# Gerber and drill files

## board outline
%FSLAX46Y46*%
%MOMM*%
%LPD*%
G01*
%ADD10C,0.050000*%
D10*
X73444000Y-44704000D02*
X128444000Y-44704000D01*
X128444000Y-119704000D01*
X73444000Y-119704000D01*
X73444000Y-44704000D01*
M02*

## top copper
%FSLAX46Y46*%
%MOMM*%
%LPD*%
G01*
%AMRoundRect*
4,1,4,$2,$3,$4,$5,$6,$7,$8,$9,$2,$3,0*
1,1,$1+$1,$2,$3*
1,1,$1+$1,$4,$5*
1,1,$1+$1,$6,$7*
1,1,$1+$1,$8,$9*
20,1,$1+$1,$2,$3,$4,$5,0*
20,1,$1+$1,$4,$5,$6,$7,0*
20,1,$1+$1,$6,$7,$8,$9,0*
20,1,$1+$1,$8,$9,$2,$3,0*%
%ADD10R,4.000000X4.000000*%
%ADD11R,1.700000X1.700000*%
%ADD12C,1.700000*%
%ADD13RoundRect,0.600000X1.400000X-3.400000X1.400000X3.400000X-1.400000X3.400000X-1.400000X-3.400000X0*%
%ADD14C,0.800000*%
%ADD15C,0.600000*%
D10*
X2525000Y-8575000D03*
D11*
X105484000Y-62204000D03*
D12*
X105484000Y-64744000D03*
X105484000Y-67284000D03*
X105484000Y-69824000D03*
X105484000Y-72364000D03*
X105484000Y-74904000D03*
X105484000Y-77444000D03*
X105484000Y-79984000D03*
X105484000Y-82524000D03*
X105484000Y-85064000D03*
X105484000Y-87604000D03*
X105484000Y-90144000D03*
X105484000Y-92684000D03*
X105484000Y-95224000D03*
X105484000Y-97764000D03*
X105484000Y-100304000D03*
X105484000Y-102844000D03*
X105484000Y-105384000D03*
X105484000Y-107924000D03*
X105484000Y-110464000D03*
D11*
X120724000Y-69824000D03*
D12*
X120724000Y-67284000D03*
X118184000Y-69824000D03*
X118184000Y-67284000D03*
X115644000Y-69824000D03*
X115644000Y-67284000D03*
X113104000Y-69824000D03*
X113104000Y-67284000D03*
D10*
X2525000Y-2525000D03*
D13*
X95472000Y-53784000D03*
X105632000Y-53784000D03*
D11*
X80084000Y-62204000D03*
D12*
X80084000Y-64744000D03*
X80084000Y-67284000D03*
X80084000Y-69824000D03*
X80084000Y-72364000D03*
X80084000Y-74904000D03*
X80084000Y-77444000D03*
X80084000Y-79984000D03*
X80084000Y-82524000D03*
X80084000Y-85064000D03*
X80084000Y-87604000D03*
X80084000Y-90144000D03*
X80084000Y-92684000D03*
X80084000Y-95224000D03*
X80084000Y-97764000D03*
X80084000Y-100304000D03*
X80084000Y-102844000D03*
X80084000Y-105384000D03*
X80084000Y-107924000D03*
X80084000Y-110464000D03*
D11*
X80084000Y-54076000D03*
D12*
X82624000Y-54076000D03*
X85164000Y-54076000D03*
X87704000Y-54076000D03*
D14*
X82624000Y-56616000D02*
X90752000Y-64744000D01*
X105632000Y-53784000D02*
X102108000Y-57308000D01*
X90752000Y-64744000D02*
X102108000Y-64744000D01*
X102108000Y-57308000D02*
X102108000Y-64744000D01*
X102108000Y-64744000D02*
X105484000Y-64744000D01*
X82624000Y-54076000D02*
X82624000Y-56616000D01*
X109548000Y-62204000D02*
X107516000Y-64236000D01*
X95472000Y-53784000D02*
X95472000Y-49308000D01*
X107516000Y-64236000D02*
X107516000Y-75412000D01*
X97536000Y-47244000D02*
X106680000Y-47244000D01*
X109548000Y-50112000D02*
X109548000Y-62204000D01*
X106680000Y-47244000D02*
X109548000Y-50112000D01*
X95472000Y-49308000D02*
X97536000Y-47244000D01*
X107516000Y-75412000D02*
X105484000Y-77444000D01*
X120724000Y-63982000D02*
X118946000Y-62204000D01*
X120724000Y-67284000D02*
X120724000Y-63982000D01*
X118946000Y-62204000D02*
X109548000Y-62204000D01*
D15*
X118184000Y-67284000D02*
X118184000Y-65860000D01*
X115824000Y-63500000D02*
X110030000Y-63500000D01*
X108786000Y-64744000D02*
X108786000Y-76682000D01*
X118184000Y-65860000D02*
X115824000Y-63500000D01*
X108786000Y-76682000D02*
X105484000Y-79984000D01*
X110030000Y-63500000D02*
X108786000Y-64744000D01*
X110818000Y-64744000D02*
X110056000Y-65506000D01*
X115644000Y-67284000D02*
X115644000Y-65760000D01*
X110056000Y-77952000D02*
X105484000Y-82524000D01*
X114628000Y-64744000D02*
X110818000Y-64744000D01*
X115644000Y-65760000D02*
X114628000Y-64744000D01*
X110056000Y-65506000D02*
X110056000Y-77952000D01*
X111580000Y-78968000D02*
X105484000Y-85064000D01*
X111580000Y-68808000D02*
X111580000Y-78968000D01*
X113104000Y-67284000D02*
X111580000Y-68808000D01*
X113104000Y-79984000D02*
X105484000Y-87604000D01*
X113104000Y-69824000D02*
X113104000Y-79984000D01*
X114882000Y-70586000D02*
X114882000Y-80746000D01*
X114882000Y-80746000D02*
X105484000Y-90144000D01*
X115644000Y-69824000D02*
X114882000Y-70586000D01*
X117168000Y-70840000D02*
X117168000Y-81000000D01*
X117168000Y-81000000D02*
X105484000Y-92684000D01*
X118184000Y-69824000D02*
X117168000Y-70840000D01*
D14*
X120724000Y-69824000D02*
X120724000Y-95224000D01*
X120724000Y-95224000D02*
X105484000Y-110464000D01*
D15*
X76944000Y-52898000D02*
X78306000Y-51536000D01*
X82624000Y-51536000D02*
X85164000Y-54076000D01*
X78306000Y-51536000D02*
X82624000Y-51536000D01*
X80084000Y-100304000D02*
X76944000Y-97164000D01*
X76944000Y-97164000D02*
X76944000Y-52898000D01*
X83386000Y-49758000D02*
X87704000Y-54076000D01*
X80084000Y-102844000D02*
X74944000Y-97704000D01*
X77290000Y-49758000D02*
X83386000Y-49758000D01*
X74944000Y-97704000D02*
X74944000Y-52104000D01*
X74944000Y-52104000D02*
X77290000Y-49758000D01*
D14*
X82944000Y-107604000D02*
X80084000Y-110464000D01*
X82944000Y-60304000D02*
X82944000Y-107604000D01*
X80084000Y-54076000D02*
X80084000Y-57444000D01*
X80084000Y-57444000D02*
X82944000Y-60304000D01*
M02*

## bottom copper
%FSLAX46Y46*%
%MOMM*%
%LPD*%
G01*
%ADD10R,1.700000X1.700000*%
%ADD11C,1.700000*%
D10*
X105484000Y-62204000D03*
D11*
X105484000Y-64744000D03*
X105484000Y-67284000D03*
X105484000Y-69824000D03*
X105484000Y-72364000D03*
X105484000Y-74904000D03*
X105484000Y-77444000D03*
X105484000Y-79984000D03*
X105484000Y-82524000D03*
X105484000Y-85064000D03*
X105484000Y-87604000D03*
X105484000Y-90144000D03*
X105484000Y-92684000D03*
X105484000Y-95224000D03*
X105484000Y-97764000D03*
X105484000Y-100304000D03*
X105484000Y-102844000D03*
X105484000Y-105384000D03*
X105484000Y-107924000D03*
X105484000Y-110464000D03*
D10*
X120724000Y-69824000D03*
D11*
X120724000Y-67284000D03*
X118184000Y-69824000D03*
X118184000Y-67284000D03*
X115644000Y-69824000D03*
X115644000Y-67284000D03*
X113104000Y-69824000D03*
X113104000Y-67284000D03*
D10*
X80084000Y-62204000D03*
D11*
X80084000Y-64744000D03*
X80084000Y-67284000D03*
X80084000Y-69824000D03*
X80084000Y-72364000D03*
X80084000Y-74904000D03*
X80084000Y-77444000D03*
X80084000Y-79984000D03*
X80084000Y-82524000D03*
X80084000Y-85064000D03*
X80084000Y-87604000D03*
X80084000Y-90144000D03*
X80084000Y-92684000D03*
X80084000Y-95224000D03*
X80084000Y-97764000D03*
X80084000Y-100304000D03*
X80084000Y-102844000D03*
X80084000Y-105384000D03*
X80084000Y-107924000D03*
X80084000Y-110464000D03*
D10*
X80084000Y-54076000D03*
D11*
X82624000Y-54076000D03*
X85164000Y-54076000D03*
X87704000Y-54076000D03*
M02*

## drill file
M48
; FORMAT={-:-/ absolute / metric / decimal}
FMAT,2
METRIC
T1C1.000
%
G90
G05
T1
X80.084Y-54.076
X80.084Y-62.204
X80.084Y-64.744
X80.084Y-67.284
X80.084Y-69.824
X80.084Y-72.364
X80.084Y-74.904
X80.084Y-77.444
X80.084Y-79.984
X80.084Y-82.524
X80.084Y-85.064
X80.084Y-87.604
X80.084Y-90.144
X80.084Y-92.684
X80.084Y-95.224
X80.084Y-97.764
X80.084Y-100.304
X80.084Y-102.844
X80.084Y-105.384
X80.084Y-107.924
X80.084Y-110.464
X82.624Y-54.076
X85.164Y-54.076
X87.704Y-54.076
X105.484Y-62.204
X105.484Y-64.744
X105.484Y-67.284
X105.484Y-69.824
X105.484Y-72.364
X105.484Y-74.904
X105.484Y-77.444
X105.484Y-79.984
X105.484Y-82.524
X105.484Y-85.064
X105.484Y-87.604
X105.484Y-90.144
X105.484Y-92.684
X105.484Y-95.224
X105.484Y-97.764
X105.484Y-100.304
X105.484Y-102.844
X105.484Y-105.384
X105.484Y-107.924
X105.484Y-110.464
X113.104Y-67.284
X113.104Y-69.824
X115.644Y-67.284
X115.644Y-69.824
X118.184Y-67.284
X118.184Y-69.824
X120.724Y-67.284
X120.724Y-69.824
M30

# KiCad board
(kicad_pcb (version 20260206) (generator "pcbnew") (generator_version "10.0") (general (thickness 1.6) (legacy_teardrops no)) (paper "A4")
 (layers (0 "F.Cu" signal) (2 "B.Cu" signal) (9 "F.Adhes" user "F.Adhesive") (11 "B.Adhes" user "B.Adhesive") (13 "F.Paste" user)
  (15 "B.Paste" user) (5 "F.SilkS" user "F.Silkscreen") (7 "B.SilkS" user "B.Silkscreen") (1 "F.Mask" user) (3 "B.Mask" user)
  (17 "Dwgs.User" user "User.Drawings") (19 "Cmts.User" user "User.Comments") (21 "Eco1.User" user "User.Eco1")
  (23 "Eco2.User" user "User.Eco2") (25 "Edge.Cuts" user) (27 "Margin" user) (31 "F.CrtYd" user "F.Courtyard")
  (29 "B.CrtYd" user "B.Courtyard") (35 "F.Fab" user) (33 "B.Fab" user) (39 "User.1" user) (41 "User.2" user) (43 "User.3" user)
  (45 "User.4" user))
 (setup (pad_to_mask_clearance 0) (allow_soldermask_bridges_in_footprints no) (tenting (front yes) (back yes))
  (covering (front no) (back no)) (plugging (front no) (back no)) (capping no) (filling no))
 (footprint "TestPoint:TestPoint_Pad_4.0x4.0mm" (layer "F.Cu") (at 2.525 8.575)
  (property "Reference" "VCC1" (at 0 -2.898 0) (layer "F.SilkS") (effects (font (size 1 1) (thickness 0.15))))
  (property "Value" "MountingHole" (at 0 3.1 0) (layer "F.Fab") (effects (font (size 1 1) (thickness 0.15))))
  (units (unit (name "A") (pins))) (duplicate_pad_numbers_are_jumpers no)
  (pad "1" smd rect (at 0 0) (size 4 4) (layers "F.Cu" "F.Mask")))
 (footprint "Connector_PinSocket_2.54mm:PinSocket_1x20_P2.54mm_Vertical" (layer "F.Cu") (at 105.484 62.204)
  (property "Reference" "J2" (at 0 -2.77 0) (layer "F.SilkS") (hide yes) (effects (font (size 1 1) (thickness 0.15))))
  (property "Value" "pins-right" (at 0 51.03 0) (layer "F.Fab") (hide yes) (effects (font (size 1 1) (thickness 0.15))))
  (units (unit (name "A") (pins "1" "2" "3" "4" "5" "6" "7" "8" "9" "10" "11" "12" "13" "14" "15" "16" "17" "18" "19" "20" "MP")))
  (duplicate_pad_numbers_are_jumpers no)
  (pad "1" thru_hole rect (at 0 0) (size 1.7 1.7) (drill 1) (layers "*.Cu" "*.Mask") (remove_unused_layers no)
   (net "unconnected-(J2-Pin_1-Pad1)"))
  (pad "2" thru_hole circle (at 0 2.54) (size 1.7 1.7) (drill 1) (layers "*.Cu" "*.Mask") (remove_unused_layers no) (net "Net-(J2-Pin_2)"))
  (pad "3" thru_hole circle (at 0 5.08) (size 1.7 1.7) (drill 1) (layers "*.Cu" "*.Mask") (remove_unused_layers no)
   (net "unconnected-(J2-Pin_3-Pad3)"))
  (pad "4" thru_hole circle (at 0 7.62) (size 1.7 1.7) (drill 1) (layers "*.Cu" "*.Mask") (remove_unused_layers no)
   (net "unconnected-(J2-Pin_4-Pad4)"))
  (pad "5" thru_hole circle (at 0 10.16) (size 1.7 1.7) (drill 1) (layers "*.Cu" "*.Mask") (remove_unused_layers no)
   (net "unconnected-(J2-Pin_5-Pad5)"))
  (pad "6" thru_hole circle (at 0 12.7) (size 1.7 1.7) (drill 1) (layers "*.Cu" "*.Mask") (remove_unused_layers no)
   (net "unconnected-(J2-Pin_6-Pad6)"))
  (pad "7" thru_hole circle (at 0 15.24) (size 1.7 1.7) (drill 1) (layers "*.Cu" "*.Mask") (remove_unused_layers no) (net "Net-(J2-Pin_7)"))
  (pad "8" thru_hole circle (at 0 17.78) (size 1.7 1.7) (drill 1) (layers "*.Cu" "*.Mask") (remove_unused_layers no) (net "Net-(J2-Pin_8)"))
  (pad "9" thru_hole circle (at 0 20.32) (size 1.7 1.7) (drill 1) (layers "*.Cu" "*.Mask") (remove_unused_layers no) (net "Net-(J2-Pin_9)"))
  (pad "10" thru_hole circle (at 0 22.86) (size 1.7 1.7) (drill 1) (layers "*.Cu" "*.Mask") (remove_unused_layers no)
   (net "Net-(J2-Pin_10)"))
  (pad "11" thru_hole circle (at 0 25.4) (size 1.7 1.7) (drill 1) (layers "*.Cu" "*.Mask") (remove_unused_layers no) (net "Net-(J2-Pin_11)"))
  (pad "12" thru_hole circle (at 0 27.94) (size 1.7 1.7) (drill 1) (layers "*.Cu" "*.Mask") (remove_unused_layers no)
   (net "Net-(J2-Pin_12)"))
  (pad "13" thru_hole circle (at 0 30.48) (size 1.7 1.7) (drill 1) (layers "*.Cu" "*.Mask") (remove_unused_layers no)
   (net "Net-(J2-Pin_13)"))
  (pad "14" thru_hole circle (at 0 33.02) (size 1.7 1.7) (drill 1) (layers "*.Cu" "*.Mask") (remove_unused_layers no)
   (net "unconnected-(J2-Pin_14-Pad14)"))
  (pad "15" thru_hole circle (at 0 35.56) (size 1.7 1.7) (drill 1) (layers "*.Cu" "*.Mask") (remove_unused_layers no)
   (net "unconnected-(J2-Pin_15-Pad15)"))
  (pad "16" thru_hole circle (at 0 38.1) (size 1.7 1.7) (drill 1) (layers "*.Cu" "*.Mask") (remove_unused_layers no)
   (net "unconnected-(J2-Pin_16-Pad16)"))
  (pad "17" thru_hole circle (at 0 40.64) (size 1.7 1.7) (drill 1) (layers "*.Cu" "*.Mask") (remove_unused_layers no)
   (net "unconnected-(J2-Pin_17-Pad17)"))
  (pad "18" thru_hole circle (at 0 43.18) (size 1.7 1.7) (drill 1) (layers "*.Cu" "*.Mask") (remove_unused_layers no)
   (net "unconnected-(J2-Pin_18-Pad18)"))
  (pad "19" thru_hole circle (at 0 45.72) (size 1.7 1.7) (drill 1) (layers "*.Cu" "*.Mask") (remove_unused_layers no)
   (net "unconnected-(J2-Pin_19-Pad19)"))
  (pad "20" thru_hole circle (at 0 48.26) (size 1.7 1.7) (drill 1) (layers "*.Cu" "*.Mask") (remove_unused_layers no)
   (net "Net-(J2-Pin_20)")))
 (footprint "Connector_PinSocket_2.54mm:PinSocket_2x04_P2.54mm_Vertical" (layer "F.Cu") (at 120.724 69.824 -90)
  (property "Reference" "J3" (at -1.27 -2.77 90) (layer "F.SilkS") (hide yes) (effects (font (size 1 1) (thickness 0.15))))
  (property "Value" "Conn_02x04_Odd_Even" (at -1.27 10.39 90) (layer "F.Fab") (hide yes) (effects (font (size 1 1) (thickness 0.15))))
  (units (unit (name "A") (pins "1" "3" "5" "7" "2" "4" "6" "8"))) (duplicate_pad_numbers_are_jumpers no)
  (pad "1" thru_hole rect (at 0 0 270) (size 1.7 1.7) (drill 1) (layers "*.Cu" "*.Mask") (remove_unused_layers no) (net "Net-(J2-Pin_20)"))
  (pad "2" thru_hole circle (at -2.54 0 270) (size 1.7 1.7) (drill 1) (layers "*.Cu" "*.Mask") (remove_unused_layers no)
   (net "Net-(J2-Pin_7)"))
  (pad "3" thru_hole circle (at 0 2.54 270) (size 1.7 1.7) (drill 1) (layers "*.Cu" "*.Mask") (remove_unused_layers no)
   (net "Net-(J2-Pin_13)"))
  (pad "4" thru_hole circle (at -2.54 2.54 270) (size 1.7 1.7) (drill 1) (layers "*.Cu" "*.Mask") (remove_unused_layers no)
   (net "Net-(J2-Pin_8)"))
  (pad "5" thru_hole circle (at 0 5.08 270) (size 1.7 1.7) (drill 1) (layers "*.Cu" "*.Mask") (remove_unused_layers no)
   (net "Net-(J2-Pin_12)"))
  (pad "6" thru_hole circle (at -2.54 5.08 270) (size 1.7 1.7) (drill 1) (layers "*.Cu" "*.Mask") (remove_unused_layers no)
   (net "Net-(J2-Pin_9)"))
  (pad "7" thru_hole circle (at 0 7.62 270) (size 1.7 1.7) (drill 1) (layers "*.Cu" "*.Mask") (remove_unused_layers no)
   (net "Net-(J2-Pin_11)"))
  (pad "8" thru_hole circle (at -2.54 7.62 270) (size 1.7 1.7) (drill 1) (layers "*.Cu" "*.Mask") (remove_unused_layers no)
   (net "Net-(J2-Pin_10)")))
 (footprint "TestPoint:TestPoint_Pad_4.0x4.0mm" (layer "F.Cu") (at 2.525 2.525)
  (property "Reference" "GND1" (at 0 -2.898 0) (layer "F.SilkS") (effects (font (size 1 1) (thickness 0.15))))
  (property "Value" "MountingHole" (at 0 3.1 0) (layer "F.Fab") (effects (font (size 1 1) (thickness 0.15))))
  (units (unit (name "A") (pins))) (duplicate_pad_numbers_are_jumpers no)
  (pad "1" smd rect (at 0 0) (size 4 4) (layers "F.Cu" "F.Mask")))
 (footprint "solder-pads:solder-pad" (layer "F.Cu") (at 100.552 53.784)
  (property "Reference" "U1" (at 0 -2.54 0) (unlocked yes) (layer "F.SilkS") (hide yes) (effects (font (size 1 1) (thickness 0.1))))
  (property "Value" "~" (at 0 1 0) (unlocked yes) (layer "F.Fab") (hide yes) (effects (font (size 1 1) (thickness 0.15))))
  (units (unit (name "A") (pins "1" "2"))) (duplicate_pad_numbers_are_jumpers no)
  (pad "1" smd roundrect (at -5.08 0 90) (size 8 4) (layers "F.Cu" "F.Mask" "F.Paste") (roundrect_rratio 0.15) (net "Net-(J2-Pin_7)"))
  (pad "2" smd roundrect (at 5.08 0 90) (size 8 4) (layers "F.Cu" "F.Mask" "F.Paste") (roundrect_rratio 0.15) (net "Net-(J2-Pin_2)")))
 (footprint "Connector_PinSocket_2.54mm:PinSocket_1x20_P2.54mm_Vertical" (layer "F.Cu") (at 80.084 62.204)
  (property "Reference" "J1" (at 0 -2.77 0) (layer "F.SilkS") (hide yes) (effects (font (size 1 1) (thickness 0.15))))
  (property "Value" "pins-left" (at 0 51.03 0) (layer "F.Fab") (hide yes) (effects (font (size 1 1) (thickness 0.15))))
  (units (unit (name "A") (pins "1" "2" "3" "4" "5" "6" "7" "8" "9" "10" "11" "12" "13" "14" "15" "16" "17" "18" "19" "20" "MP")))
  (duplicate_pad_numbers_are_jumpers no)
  (pad "1" thru_hole rect (at 0 0) (size 1.7 1.7) (drill 1) (layers "*.Cu" "*.Mask") (remove_unused_layers no)
   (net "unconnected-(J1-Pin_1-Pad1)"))
  (pad "2" thru_hole circle (at 0 2.54) (size 1.7 1.7) (drill 1) (layers "*.Cu" "*.Mask") (remove_unused_layers no)
   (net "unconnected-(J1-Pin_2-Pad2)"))
  (pad "3" thru_hole circle (at 0 5.08) (size 1.7 1.7) (drill 1) (layers "*.Cu" "*.Mask") (remove_unused_layers no)
   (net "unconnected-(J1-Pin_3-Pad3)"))
  (pad "4" thru_hole circle (at 0 7.62) (size 1.7 1.7) (drill 1) (layers "*.Cu" "*.Mask") (remove_unused_layers no)
   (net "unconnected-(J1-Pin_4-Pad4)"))
  (pad "5" thru_hole circle (at 0 10.16) (size 1.7 1.7) (drill 1) (layers "*.Cu" "*.Mask") (remove_unused_layers no)
   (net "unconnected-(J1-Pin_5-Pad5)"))
  (pad "6" thru_hole circle (at 0 12.7) (size 1.7 1.7) (drill 1) (layers "*.Cu" "*.Mask") (remove_unused_layers no)
   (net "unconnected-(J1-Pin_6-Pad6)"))
  (pad "7" thru_hole circle (at 0 15.24) (size 1.7 1.7) (drill 1) (layers "*.Cu" "*.Mask") (remove_unused_layers no)
   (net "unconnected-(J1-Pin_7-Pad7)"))
  (pad "8" thru_hole circle (at 0 17.78) (size 1.7 1.7) (drill 1) (layers "*.Cu" "*.Mask") (remove_unused_layers no)
   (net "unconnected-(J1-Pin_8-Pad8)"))
  (pad "9" thru_hole circle (at 0 20.32) (size 1.7 1.7) (drill 1) (layers "*.Cu" "*.Mask") (remove_unused_layers no)
   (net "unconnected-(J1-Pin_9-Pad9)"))
  (pad "10" thru_hole circle (at 0 22.86) (size 1.7 1.7) (drill 1) (layers "*.Cu" "*.Mask") (remove_unused_layers no)
   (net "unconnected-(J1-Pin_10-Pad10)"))
  (pad "11" thru_hole circle (at 0 25.4) (size 1.7 1.7) (drill 1) (layers "*.Cu" "*.Mask") (remove_unused_layers no)
   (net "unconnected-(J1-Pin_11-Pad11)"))
  (pad "12" thru_hole circle (at 0 27.94) (size 1.7 1.7) (drill 1) (layers "*.Cu" "*.Mask") (remove_unused_layers no)
   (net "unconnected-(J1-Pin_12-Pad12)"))
  (pad "13" thru_hole circle (at 0 30.48) (size 1.7 1.7) (drill 1) (layers "*.Cu" "*.Mask") (remove_unused_layers no)
   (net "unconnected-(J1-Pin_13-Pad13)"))
  (pad "14" thru_hole circle (at 0 33.02) (size 1.7 1.7) (drill 1) (layers "*.Cu" "*.Mask") (remove_unused_layers no)
   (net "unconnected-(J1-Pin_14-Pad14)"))
  (pad "15" thru_hole circle (at 0 35.56) (size 1.7 1.7) (drill 1) (layers "*.Cu" "*.Mask") (remove_unused_layers no)
   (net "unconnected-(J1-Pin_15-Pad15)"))
  (pad "16" thru_hole circle (at 0 38.1) (size 1.7 1.7) (drill 1) (layers "*.Cu" "*.Mask") (remove_unused_layers no) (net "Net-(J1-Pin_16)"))
  (pad "17" thru_hole circle (at 0 40.64) (size 1.7 1.7) (drill 1) (layers "*.Cu" "*.Mask") (remove_unused_layers no)
   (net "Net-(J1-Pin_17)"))
  (pad "18" thru_hole circle (at 0 43.18) (size 1.7 1.7) (drill 1) (layers "*.Cu" "*.Mask") (remove_unused_layers no)
   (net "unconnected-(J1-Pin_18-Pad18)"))
  (pad "19" thru_hole circle (at 0 45.72) (size 1.7 1.7) (drill 1) (layers "*.Cu" "*.Mask") (remove_unused_layers no)
   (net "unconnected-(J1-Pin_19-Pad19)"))
  (pad "20" thru_hole circle (at 0 48.26) (size 1.7 1.7) (drill 1) (layers "*.Cu" "*.Mask") (remove_unused_layers no)
   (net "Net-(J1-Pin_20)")))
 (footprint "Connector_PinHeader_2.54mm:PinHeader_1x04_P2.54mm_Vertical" (layer "F.Cu") (at 80.084 54.076 90)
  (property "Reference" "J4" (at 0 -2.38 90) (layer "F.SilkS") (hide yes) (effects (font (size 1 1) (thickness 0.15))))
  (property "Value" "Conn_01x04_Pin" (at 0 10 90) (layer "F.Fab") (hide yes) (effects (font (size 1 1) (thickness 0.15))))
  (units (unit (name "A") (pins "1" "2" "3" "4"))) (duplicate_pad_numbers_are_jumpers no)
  (pad "1" thru_hole rect (at 0 0 90) (size 1.7 1.7) (drill 1) (layers "*.Cu" "*.Mask") (remove_unused_layers no) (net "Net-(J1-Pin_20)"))
  (pad "2" thru_hole circle (at 0 2.54 90) (size 1.7 1.7) (drill 1) (layers "*.Cu" "*.Mask") (remove_unused_layers no)
   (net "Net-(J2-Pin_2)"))
  (pad "3" thru_hole circle (at 0 5.08 90) (size 1.7 1.7) (drill 1) (layers "*.Cu" "*.Mask") (remove_unused_layers no)
   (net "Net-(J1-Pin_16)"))
  (pad "4" thru_hole circle (at 0 7.62 90) (size 1.7 1.7) (drill 1) (layers "*.Cu" "*.Mask") (remove_unused_layers no)
   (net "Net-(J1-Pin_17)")))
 (gr_rect (start 73.444 44.704) (end 128.444 119.704) (stroke (width 0.05) (type default)) (fill no) (layer "Edge.Cuts"))
 (segment (start 82.624 56.616) (end 90.752 64.744) (width 0.8) (layer "F.Cu") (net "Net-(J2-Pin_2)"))
 (segment (start 105.632 53.784) (end 102.108 57.308) (width 0.8) (layer "F.Cu") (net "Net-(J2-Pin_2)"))
 (segment (start 90.752 64.744) (end 102.108 64.744) (width 0.8) (layer "F.Cu") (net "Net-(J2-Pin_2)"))
 (segment (start 102.108 57.308) (end 102.108 64.744) (width 0.8) (layer "F.Cu") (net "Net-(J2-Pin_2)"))
 (segment (start 102.108 64.744) (end 105.484 64.744) (width 0.8) (layer "F.Cu") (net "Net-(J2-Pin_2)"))
 (segment (start 82.624 54.076) (end 82.624 56.616) (width 0.8) (layer "F.Cu") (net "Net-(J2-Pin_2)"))
 (segment (start 109.548 62.204) (end 107.516 64.236) (width 0.8) (layer "F.Cu") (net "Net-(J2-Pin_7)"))
 (segment (start 95.472 53.784) (end 95.472 49.308) (width 0.8) (layer "F.Cu") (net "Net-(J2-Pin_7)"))
 (segment (start 107.516 64.236) (end 107.516 75.412) (width 0.8) (layer "F.Cu") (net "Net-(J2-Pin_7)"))
 (segment (start 97.536 47.244) (end 106.68 47.244) (width 0.8) (layer "F.Cu") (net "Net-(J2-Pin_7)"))
 (segment (start 109.548 50.112) (end 109.548 62.204) (width 0.8) (layer "F.Cu") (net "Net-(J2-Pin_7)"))
 (segment (start 106.68 47.244) (end 109.548 50.112) (width 0.8) (layer "F.Cu") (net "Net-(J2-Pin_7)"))
 (segment (start 95.472 49.308) (end 97.536 47.244) (width 0.8) (layer "F.Cu") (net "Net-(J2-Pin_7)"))
 (segment (start 107.516 75.412) (end 105.484 77.444) (width 0.8) (layer "F.Cu") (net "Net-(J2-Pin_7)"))
 (segment (start 120.724 63.982) (end 118.946 62.204) (width 0.8) (layer "F.Cu") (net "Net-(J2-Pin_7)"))
 (segment (start 120.724 67.284) (end 120.724 63.982) (width 0.8) (layer "F.Cu") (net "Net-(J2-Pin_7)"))
 (segment (start 118.946 62.204) (end 109.548 62.204) (width 0.8) (layer "F.Cu") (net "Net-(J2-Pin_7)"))
 (segment (start 118.184 67.284) (end 118.184 65.86) (width 0.6) (layer "F.Cu") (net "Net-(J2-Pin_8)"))
 (segment (start 115.824 63.5) (end 110.03 63.5) (width 0.6) (layer "F.Cu") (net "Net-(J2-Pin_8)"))
 (segment (start 108.786 64.744) (end 108.786 76.682) (width 0.6) (layer "F.Cu") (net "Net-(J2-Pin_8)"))
 (segment (start 118.184 65.86) (end 115.824 63.5) (width 0.6) (layer "F.Cu") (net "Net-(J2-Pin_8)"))
 (segment (start 108.786 76.682) (end 105.484 79.984) (width 0.6) (layer "F.Cu") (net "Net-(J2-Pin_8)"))
 (segment (start 110.03 63.5) (end 108.786 64.744) (width 0.6) (layer "F.Cu") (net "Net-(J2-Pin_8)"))
 (segment (start 110.818 64.744) (end 110.056 65.506) (width 0.6) (layer "F.Cu") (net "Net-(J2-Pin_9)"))
 (segment (start 115.644 67.284) (end 115.644 65.76) (width 0.6) (layer "F.Cu") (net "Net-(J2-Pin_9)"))
 (segment (start 110.056 77.952) (end 105.484 82.524) (width 0.6) (layer "F.Cu") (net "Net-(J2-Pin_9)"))
 (segment (start 114.628 64.744) (end 110.818 64.744) (width 0.6) (layer "F.Cu") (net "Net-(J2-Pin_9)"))
 (segment (start 115.644 65.76) (end 114.628 64.744) (width 0.6) (layer "F.Cu") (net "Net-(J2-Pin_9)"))
 (segment (start 110.056 65.506) (end 110.056 77.952) (width 0.6) (layer "F.Cu") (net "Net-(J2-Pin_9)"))
 (segment (start 111.58 78.968) (end 105.484 85.064) (width 0.6) (layer "F.Cu") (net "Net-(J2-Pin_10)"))
 (segment (start 111.58 68.808) (end 111.58 78.968) (width 0.6) (layer "F.Cu") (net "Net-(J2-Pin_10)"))
 (segment (start 113.104 67.284) (end 111.58 68.808) (width 0.6) (layer "F.Cu") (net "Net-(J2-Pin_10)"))
 (segment (start 113.104 79.984) (end 105.484 87.604) (width 0.6) (layer "F.Cu") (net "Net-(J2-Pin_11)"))
 (segment (start 113.104 69.824) (end 113.104 79.984) (width 0.6) (layer "F.Cu") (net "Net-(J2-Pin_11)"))
 (segment (start 114.882 70.586) (end 114.882 80.746) (width 0.6) (layer "F.Cu") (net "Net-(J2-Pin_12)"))
 (segment (start 114.882 80.746) (end 105.484 90.144) (width 0.6) (layer "F.Cu") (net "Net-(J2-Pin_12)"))
 (segment (start 115.644 69.824) (end 114.882 70.586) (width 0.6) (layer "F.Cu") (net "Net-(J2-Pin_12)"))
 (segment (start 117.168 70.84) (end 117.168 81) (width 0.6) (layer "F.Cu") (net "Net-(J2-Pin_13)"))
 (segment (start 117.168 81) (end 105.484 92.684) (width 0.6) (layer "F.Cu") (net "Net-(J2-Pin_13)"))
 (segment (start 118.184 69.824) (end 117.168 70.84) (width 0.6) (layer "F.Cu") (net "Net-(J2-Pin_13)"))
 (segment (start 120.724 69.824) (end 120.724 95.224) (width 0.8) (layer "F.Cu") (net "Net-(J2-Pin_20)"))
 (segment (start 120.724 95.224) (end 105.484 110.464) (width 0.8) (layer "F.Cu") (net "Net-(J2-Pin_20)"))
 (segment (start 76.944 52.898) (end 78.306 51.536) (width 0.6) (layer "F.Cu") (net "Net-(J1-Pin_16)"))
 (segment (start 82.624 51.536) (end 85.164 54.076) (width 0.6) (layer "F.Cu") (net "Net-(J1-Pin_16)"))
 (segment (start 78.306 51.536) (end 82.624 51.536) (width 0.6) (layer "F.Cu") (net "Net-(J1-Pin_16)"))
 (segment (start 80.084 100.304) (end 76.944 97.164) (width 0.6) (layer "F.Cu") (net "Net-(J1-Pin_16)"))
 (segment (start 76.944 97.164) (end 76.944 52.898) (width 0.6) (layer "F.Cu") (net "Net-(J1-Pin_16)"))
 (segment (start 83.386 49.758) (end 87.704 54.076) (width 0.6) (layer "F.Cu") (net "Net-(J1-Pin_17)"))
 (segment (start 80.084 102.844) (end 74.944 97.704) (width 0.6) (layer "F.Cu") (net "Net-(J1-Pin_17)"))
 (segment (start 77.29 49.758) (end 83.386 49.758) (width 0.6) (layer "F.Cu") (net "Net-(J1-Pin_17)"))
 (segment (start 74.944 97.704) (end 74.944 52.104) (width 0.6) (layer "F.Cu") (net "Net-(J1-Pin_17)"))
 (segment (start 74.944 52.104) (end 77.29 49.758) (width 0.6) (layer "F.Cu") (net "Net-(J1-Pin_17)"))
 (segment (start 82.944 107.604) (end 80.084 110.464) (width 0.8) (layer "F.Cu") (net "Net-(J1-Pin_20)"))
 (segment (start 82.944 60.304) (end 82.944 107.604) (width 0.8) (layer "F.Cu") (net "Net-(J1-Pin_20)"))
 (segment (start 80.084 54.076) (end 80.084 57.444) (width 0.8) (layer "F.Cu") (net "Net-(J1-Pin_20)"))
 (segment (start 80.084 57.444) (end 82.944 60.304) (width 0.8) (layer "F.Cu") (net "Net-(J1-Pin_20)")))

